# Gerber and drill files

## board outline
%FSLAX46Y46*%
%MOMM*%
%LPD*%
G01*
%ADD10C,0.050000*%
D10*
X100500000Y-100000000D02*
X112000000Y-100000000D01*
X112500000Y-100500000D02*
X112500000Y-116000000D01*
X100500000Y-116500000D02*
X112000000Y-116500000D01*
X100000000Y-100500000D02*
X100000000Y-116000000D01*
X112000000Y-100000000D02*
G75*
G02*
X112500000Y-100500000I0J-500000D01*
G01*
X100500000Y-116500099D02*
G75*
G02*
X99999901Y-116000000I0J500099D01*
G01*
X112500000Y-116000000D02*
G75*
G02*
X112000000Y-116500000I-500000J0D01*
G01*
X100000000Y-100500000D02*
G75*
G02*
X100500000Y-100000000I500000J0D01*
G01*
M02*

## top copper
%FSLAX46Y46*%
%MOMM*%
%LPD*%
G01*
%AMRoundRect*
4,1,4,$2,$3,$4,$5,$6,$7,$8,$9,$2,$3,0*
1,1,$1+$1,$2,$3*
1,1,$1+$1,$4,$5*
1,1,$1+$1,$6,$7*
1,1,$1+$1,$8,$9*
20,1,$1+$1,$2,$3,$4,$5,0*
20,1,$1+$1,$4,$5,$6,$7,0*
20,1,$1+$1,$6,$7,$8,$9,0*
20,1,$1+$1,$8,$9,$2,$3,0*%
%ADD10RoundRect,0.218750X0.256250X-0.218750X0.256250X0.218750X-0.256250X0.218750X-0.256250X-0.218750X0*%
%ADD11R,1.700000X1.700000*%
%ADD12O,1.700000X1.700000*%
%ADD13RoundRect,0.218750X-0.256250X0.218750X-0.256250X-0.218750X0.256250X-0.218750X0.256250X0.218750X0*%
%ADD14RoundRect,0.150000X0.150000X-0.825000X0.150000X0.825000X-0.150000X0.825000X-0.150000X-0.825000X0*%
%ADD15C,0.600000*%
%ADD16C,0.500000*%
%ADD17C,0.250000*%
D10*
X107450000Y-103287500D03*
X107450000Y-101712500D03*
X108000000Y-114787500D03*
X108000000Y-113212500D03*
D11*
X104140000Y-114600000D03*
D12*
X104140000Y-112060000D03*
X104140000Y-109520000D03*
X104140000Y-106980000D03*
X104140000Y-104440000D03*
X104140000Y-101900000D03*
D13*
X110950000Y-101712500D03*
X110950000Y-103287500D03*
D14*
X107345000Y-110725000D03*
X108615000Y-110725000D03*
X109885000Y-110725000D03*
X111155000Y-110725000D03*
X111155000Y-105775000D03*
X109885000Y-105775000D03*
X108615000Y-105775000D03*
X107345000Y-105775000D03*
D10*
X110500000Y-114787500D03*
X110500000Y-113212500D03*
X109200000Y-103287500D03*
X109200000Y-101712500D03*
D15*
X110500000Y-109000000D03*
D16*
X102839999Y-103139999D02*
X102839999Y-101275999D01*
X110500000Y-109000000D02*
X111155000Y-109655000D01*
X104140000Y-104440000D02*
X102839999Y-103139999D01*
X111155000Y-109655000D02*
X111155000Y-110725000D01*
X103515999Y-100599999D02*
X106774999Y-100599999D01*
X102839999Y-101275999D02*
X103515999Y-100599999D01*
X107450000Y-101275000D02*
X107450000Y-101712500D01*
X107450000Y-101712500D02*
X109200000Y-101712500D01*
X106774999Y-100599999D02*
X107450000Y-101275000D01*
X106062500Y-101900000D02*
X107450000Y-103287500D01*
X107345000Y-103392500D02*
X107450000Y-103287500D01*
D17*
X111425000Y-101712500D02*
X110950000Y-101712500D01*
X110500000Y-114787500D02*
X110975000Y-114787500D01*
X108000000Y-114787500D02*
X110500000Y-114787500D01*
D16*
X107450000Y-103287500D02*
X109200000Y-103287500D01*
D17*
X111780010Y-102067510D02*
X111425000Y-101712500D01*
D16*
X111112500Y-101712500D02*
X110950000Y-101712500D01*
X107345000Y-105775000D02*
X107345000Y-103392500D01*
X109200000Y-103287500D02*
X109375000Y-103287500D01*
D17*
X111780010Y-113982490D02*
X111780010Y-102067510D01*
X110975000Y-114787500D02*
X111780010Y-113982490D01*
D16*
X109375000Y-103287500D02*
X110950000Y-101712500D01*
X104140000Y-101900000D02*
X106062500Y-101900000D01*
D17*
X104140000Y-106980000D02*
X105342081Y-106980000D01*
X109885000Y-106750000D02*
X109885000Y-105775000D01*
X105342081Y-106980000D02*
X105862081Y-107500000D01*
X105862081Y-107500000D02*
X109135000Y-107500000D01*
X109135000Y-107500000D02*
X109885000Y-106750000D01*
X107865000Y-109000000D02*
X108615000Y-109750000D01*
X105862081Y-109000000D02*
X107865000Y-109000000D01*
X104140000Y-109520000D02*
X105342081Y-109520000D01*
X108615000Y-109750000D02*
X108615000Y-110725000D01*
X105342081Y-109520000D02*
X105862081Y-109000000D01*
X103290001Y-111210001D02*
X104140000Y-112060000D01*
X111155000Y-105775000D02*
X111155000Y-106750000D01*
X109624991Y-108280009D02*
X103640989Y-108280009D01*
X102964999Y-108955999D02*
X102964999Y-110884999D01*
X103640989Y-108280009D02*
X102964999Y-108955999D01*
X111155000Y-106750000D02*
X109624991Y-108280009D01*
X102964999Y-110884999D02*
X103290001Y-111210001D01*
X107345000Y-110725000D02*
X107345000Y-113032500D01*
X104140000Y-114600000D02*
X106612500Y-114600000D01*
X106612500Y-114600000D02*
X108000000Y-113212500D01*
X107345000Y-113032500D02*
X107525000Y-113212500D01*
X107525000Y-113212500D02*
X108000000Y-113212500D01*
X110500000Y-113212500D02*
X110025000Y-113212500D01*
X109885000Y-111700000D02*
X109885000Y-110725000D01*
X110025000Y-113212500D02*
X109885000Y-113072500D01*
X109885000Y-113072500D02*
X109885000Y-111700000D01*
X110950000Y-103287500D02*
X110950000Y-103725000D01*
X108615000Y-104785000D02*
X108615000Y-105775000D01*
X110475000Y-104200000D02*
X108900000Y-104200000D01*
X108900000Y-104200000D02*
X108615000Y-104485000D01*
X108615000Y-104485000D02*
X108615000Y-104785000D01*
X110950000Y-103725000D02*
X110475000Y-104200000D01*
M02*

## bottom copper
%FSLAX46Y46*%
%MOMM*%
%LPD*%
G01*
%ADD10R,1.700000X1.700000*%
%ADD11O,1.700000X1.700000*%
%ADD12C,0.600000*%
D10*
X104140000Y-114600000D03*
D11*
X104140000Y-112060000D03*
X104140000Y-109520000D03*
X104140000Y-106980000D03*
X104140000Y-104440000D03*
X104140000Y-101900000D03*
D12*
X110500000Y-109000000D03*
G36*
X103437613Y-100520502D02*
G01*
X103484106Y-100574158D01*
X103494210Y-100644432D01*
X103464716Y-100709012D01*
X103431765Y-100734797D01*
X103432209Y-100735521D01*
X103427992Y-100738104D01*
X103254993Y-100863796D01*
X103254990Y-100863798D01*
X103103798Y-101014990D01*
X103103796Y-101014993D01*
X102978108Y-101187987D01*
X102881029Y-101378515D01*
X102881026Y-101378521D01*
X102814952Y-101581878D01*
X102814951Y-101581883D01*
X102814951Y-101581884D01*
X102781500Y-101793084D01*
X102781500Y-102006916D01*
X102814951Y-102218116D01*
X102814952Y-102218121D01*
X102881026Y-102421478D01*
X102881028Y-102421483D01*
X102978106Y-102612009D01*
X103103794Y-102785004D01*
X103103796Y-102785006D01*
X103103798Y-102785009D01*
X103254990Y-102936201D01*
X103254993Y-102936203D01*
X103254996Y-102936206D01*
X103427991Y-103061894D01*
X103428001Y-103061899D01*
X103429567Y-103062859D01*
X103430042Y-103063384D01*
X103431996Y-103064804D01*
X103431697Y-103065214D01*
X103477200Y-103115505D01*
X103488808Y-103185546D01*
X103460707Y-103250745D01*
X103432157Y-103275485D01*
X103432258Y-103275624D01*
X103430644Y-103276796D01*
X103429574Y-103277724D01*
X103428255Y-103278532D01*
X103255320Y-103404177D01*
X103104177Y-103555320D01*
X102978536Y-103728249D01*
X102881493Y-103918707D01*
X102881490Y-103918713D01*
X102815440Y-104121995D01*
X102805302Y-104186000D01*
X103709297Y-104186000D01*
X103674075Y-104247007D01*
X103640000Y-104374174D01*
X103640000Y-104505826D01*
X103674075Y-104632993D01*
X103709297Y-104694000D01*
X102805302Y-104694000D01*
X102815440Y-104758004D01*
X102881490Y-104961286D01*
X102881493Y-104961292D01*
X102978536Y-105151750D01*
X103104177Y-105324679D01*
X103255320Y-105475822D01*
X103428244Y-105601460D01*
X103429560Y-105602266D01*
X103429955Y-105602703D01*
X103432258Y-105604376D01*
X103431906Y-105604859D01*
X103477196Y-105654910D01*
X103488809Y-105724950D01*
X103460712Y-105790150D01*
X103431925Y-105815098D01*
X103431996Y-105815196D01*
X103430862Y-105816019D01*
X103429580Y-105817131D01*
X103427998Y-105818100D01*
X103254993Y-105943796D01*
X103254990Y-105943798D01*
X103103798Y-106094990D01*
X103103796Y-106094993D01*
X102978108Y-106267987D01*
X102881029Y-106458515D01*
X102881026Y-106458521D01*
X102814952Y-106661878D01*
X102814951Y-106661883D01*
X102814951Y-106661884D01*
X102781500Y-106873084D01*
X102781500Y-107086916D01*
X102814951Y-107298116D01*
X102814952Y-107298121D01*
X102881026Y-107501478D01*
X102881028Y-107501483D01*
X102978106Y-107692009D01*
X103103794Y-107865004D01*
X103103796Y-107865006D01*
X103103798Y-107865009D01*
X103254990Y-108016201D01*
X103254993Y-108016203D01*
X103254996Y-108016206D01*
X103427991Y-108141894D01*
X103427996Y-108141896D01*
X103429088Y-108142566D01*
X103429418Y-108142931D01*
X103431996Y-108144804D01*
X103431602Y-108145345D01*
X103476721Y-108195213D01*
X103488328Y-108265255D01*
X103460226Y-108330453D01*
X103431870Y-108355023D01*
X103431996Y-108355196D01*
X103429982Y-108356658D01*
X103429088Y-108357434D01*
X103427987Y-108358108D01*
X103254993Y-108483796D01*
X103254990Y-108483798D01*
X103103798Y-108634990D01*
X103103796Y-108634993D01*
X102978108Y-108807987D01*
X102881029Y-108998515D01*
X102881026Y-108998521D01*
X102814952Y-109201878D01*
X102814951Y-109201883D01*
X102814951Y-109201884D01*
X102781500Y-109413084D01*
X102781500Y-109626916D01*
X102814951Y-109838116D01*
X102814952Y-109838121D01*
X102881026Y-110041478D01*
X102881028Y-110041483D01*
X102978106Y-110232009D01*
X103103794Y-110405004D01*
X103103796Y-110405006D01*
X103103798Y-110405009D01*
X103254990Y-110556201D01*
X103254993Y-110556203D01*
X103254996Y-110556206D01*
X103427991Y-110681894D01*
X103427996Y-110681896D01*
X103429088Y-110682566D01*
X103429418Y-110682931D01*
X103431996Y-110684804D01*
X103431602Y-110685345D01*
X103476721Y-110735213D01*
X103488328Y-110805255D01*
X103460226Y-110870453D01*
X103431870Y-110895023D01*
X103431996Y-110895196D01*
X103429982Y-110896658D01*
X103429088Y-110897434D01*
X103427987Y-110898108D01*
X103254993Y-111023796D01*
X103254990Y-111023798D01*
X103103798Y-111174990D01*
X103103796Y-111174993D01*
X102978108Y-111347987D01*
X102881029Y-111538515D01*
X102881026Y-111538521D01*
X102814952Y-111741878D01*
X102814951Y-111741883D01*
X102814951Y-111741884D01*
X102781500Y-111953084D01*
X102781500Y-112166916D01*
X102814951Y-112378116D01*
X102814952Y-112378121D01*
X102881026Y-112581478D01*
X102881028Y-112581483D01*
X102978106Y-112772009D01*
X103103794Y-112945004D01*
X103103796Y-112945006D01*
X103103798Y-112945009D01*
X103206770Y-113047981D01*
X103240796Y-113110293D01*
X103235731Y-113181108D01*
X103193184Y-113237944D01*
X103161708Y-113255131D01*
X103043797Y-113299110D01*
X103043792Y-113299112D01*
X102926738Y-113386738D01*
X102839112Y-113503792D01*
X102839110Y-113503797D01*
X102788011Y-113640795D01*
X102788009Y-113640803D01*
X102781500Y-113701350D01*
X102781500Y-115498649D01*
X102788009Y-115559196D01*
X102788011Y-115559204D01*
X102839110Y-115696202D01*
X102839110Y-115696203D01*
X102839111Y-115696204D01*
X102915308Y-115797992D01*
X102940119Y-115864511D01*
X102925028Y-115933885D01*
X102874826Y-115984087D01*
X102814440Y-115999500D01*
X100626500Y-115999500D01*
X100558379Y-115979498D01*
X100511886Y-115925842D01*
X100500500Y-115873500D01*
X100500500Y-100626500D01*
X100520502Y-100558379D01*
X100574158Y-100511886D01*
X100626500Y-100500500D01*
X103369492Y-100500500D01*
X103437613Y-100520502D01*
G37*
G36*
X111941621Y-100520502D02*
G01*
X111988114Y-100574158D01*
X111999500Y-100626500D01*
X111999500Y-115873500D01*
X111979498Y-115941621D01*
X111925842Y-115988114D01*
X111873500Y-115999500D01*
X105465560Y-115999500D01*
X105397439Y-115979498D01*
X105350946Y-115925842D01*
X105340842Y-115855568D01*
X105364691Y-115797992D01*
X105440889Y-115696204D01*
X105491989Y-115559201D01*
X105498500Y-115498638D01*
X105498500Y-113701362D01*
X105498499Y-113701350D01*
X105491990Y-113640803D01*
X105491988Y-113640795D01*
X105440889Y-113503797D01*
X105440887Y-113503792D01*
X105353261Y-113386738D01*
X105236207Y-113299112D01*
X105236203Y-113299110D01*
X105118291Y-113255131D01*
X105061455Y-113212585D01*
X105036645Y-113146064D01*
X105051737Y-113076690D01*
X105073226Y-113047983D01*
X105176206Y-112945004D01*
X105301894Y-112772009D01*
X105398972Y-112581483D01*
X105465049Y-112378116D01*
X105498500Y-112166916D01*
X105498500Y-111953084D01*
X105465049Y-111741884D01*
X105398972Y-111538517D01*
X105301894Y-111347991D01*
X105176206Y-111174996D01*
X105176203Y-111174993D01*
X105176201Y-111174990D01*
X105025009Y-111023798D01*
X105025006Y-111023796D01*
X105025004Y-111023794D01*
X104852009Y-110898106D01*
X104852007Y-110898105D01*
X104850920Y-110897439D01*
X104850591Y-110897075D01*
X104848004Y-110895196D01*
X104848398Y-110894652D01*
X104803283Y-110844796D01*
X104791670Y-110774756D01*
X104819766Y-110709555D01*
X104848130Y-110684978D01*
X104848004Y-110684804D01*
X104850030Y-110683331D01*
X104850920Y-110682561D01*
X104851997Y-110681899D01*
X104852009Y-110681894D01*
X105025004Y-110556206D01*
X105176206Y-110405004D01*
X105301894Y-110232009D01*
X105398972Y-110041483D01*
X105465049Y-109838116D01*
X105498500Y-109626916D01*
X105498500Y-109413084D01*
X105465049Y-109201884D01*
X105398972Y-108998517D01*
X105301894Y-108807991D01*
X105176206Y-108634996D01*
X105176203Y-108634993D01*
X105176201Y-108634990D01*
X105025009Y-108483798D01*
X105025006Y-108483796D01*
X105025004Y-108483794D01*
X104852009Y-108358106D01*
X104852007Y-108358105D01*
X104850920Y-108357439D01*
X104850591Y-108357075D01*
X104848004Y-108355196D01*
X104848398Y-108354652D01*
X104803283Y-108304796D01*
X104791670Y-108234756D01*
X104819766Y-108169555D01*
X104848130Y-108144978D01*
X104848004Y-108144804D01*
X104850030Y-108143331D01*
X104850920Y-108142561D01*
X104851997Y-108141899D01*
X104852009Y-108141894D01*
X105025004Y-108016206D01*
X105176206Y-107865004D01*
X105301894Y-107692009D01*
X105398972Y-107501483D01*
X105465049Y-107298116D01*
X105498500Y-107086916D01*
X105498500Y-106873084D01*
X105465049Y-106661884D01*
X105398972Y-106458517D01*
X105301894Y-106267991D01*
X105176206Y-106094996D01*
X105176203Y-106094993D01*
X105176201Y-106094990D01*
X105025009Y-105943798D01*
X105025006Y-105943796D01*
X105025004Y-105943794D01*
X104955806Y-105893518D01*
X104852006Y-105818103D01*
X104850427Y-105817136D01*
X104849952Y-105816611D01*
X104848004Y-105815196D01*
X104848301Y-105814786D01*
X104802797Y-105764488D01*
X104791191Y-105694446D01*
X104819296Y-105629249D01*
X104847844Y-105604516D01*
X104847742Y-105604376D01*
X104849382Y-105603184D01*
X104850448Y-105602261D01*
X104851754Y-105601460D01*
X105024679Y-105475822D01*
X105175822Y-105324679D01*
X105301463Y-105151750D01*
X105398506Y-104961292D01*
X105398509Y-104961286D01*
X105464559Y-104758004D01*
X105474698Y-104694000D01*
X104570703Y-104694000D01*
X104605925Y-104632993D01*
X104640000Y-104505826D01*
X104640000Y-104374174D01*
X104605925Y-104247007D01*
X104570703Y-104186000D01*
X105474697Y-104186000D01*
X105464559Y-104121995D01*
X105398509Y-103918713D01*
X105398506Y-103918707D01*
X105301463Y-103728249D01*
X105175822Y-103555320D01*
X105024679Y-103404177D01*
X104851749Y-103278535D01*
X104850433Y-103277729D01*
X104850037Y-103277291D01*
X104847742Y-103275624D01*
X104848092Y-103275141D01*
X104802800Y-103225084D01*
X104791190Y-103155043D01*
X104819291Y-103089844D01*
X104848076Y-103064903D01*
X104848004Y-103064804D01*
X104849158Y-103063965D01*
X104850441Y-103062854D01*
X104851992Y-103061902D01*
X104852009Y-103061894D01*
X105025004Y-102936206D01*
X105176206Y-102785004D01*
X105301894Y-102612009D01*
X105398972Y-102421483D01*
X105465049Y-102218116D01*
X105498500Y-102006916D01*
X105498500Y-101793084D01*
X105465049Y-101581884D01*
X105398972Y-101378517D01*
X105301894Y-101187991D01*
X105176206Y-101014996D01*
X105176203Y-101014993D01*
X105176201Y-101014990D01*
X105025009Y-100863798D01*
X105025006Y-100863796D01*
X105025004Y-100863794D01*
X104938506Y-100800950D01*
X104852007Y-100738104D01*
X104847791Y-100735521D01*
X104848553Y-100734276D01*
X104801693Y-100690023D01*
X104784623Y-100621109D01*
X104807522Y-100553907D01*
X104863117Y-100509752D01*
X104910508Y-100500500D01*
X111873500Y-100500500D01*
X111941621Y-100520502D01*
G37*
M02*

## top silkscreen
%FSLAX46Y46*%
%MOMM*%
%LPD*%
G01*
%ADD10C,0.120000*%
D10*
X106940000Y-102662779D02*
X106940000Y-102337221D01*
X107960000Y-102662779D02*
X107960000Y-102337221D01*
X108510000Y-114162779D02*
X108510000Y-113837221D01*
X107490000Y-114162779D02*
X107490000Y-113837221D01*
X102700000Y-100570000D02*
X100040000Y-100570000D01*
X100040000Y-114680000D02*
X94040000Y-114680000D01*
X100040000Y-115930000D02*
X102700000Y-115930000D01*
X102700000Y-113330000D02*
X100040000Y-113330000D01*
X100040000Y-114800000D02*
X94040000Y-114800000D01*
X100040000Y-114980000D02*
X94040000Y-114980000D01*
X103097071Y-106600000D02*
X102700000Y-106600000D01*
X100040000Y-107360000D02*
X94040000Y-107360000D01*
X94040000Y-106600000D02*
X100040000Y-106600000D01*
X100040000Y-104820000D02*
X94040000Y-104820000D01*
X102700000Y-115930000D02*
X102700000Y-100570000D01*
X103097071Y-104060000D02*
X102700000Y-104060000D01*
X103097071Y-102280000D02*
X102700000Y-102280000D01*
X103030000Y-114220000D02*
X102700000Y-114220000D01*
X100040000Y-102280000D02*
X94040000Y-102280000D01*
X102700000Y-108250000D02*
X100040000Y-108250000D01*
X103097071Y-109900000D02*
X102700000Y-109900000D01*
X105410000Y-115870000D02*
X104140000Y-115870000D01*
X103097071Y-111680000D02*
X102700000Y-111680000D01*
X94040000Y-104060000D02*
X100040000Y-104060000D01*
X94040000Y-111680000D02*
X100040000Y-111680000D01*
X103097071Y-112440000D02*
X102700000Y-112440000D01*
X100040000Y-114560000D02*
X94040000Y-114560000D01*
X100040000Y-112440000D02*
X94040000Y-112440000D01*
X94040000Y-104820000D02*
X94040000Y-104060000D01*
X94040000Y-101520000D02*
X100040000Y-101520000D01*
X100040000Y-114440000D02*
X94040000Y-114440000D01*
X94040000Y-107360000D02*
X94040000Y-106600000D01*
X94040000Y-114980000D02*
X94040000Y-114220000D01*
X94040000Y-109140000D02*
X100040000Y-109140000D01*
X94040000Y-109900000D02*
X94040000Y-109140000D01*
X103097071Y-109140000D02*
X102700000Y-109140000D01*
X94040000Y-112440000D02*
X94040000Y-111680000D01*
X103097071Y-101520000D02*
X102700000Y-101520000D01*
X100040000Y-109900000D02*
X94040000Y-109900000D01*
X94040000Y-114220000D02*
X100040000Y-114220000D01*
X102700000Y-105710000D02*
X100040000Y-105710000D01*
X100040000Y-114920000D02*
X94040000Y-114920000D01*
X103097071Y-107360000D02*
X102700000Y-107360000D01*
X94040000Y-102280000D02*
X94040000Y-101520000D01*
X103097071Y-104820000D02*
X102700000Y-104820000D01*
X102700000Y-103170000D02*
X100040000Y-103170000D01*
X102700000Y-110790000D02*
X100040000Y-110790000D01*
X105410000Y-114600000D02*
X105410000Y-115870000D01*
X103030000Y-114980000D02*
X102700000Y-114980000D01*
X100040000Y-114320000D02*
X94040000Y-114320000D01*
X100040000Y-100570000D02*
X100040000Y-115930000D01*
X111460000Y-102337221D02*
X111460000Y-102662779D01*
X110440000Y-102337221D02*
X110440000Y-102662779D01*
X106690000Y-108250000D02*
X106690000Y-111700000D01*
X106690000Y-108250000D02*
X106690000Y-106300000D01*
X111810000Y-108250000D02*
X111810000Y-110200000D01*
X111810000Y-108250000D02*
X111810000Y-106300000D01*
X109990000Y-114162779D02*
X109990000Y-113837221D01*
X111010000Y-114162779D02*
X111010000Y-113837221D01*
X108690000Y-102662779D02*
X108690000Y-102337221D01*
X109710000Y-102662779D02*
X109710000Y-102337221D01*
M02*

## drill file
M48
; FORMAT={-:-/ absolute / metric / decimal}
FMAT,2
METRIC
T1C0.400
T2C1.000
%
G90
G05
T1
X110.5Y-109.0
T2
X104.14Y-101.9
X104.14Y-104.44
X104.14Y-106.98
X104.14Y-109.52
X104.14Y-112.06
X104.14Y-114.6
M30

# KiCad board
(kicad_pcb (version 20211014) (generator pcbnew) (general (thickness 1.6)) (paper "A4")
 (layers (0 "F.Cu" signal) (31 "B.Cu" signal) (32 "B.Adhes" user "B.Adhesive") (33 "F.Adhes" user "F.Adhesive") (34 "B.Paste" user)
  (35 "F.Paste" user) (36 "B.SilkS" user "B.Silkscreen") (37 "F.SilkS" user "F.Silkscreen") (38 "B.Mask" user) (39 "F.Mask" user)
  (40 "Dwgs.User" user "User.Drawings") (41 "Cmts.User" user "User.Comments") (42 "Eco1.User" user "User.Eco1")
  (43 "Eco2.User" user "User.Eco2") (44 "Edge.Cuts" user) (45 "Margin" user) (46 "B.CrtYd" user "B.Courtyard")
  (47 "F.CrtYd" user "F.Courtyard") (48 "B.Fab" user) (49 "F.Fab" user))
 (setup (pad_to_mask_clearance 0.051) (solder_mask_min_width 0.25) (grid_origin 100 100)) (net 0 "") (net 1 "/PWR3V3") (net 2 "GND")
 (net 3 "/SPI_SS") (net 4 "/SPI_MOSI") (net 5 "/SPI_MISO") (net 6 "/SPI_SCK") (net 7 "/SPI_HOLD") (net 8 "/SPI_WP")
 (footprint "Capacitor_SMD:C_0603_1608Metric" (layer "F.Cu") (at 107.45 102.5 90)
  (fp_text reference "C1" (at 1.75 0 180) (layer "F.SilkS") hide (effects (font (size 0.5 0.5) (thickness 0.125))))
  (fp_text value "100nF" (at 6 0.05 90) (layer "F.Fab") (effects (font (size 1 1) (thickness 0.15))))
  (fp_line (start -0.162779 -0.51) (end 0.162779 -0.51) (layer "F.SilkS") (width 0.12))
  (fp_line (start -0.162779 0.51) (end 0.162779 0.51) (layer "F.SilkS") (width 0.12))
  (pad "1" smd roundrect locked (at -0.7875 0 90) (size 0.875 0.95) (layers "F.Cu" "F.Paste" "F.Mask") (roundrect_rratio 0.25)
   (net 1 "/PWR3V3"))
  (pad "2" smd roundrect locked (at 0.7875 0 90) (size 0.875 0.95) (layers "F.Cu" "F.Paste" "F.Mask") (roundrect_rratio 0.25) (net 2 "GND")))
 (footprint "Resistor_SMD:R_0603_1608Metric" (layer "F.Cu") (at 108 114 90)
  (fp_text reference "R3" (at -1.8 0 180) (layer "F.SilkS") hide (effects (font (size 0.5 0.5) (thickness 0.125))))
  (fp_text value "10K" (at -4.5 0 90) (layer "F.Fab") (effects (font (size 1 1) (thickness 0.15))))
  (fp_line (start -0.162779 0.51) (end 0.162779 0.51) (layer "F.SilkS") (width 0.12))
  (fp_line (start -0.162779 -0.51) (end 0.162779 -0.51) (layer "F.SilkS") (width 0.12))
  (pad "1" smd roundrect locked (at -0.7875 0 90) (size 0.875 0.95) (layers "F.Cu" "F.Paste" "F.Mask") (roundrect_rratio 0.25)
   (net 1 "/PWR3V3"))
  (pad "2" smd roundrect locked (at 0.7875 0 90) (size 0.875 0.95) (layers "F.Cu" "F.Paste" "F.Mask") (roundrect_rratio 0.25)
   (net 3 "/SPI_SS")))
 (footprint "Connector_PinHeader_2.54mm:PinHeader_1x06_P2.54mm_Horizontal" (layer "F.Cu") (at 104.14 114.6 180)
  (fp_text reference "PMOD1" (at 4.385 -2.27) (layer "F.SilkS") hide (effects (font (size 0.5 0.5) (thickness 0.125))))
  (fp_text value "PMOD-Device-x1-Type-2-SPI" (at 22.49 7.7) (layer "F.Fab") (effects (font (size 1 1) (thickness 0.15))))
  (fp_line (start 1.44 14.03) (end 4.1 14.03) (layer "F.SilkS") (width 0.12))
  (fp_line (start 4.1 -0.08) (end 10.1 -0.08) (layer "F.SilkS") (width 0.12))
  (fp_line (start 4.1 -1.33) (end 1.44 -1.33) (layer "F.SilkS") (width 0.12))
  (fp_line (start 1.44 1.27) (end 4.1 1.27) (layer "F.SilkS") (width 0.12))
  (fp_line (start 4.1 -0.2) (end 10.1 -0.2) (layer "F.SilkS") (width 0.12))
  (fp_line (start 4.1 -0.38) (end 10.1 -0.38) (layer "F.SilkS") (width 0.12))
  (fp_line (start 1.042929 8) (end 1.44 8) (layer "F.SilkS") (width 0.12))
  (fp_line (start 4.1 7.24) (end 10.1 7.24) (layer "F.SilkS") (width 0.12))
  (fp_line (start 10.1 8) (end 4.1 8) (layer "F.SilkS") (width 0.12))
  (fp_line (start 4.1 9.78) (end 10.1 9.78) (layer "F.SilkS") (width 0.12))
  (fp_line (start 1.44 -1.33) (end 1.44 14.03) (layer "F.SilkS") (width 0.12))
  (fp_line (start 1.042929 10.54) (end 1.44 10.54) (layer "F.SilkS") (width 0.12))
  (fp_line (start 1.042929 12.32) (end 1.44 12.32) (layer "F.SilkS") (width 0.12))
  (fp_line (start 1.11 0.38) (end 1.44 0.38) (layer "F.SilkS") (width 0.12))
  (fp_line (start 4.1 12.32) (end 10.1 12.32) (layer "F.SilkS") (width 0.12))
  (fp_line (start 1.44 6.35) (end 4.1 6.35) (layer "F.SilkS") (width 0.12))
  (fp_line (start 1.042929 4.7) (end 1.44 4.7) (layer "F.SilkS") (width 0.12))
  (fp_line (start -1.27 -1.27) (end 0 -1.27) (layer "F.SilkS") (width 0.12))
  (fp_line (start 1.042929 2.92) (end 1.44 2.92) (layer "F.SilkS") (width 0.12))
  (fp_line (start 10.1 10.54) (end 4.1 10.54) (layer "F.SilkS") (width 0.12))
  (fp_line (start 10.1 2.92) (end 4.1 2.92) (layer "F.SilkS") (width 0.12))
  (fp_line (start 1.042929 2.16) (end 1.44 2.16) (layer "F.SilkS") (width 0.12))
  (fp_line (start 4.1 0.04) (end 10.1 0.04) (layer "F.SilkS") (width 0.12))
  (fp_line (start 4.1 2.16) (end 10.1 2.16) (layer "F.SilkS") (width 0.12))
  (fp_line (start 10.1 9.78) (end 10.1 10.54) (layer "F.SilkS") (width 0.12))
  (fp_line (start 10.1 13.08) (end 4.1 13.08) (layer "F.SilkS") (width 0.12))
  (fp_line (start 4.1 0.16) (end 10.1 0.16) (layer "F.SilkS") (width 0.12))
  (fp_line (start 10.1 7.24) (end 10.1 8) (layer "F.SilkS") (width 0.12))
  (fp_line (start 10.1 -0.38) (end 10.1 0.38) (layer "F.SilkS") (width 0.12))
  (fp_line (start 10.1 5.46) (end 4.1 5.46) (layer "F.SilkS") (width 0.12))
  (fp_line (start 10.1 4.7) (end 10.1 5.46) (layer "F.SilkS") (width 0.12))
  (fp_line (start 1.042929 5.46) (end 1.44 5.46) (layer "F.SilkS") (width 0.12))
  (fp_line (start 10.1 2.16) (end 10.1 2.92) (layer "F.SilkS") (width 0.12))
  (fp_line (start 1.042929 13.08) (end 1.44 13.08) (layer "F.SilkS") (width 0.12))
  (fp_line (start 4.1 4.7) (end 10.1 4.7) (layer "F.SilkS") (width 0.12))
  (fp_line (start 10.1 0.38) (end 4.1 0.38) (layer "F.SilkS") (width 0.12))
  (fp_line (start 1.44 8.89) (end 4.1 8.89) (layer "F.SilkS") (width 0.12))
  (fp_line (start 4.1 -0.32) (end 10.1 -0.32) (layer "F.SilkS") (width 0.12))
  (fp_line (start 1.042929 7.24) (end 1.44 7.24) (layer "F.SilkS") (width 0.12))
  (fp_line (start 10.1 12.32) (end 10.1 13.08) (layer "F.SilkS") (width 0.12))
  (fp_line (start 1.042929 9.78) (end 1.44 9.78) (layer "F.SilkS") (width 0.12))
  (fp_line (start 1.44 11.43) (end 4.1 11.43) (layer "F.SilkS") (width 0.12))
  (fp_line (start 1.44 3.81) (end 4.1 3.81) (layer "F.SilkS") (width 0.12))
  (fp_line (start -1.27 0) (end -1.27 -1.27) (layer "F.SilkS") (width 0.12))
  (fp_line (start 1.11 -0.38) (end 1.44 -0.38) (layer "F.SilkS") (width 0.12))
  (fp_line (start 4.1 0.28) (end 10.1 0.28) (layer "F.SilkS") (width 0.12))
  (fp_line (start 4.1 14.03) (end 4.1 -1.33) (layer "F.SilkS") (width 0.12))
  (pad "1" thru_hole rect locked (at 0 0 180) (size 1.7 1.7) (drill 1) (layers *.Cu *.Mask) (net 3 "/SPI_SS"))
  (pad "2" thru_hole oval locked (at 0 2.54 180) (size 1.7 1.7) (drill 1) (layers *.Cu *.Mask) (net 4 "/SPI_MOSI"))
  (pad "3" thru_hole oval locked (at 0 5.08 180) (size 1.7 1.7) (drill 1) (layers *.Cu *.Mask) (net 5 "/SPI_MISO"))
  (pad "4" thru_hole oval locked (at 0 7.62 180) (size 1.7 1.7) (drill 1) (layers *.Cu *.Mask) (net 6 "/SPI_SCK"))
  (pad "5" thru_hole oval locked (at 0 10.16 180) (size 1.7 1.7) (drill 1) (layers *.Cu *.Mask) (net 2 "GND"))
  (pad "6" thru_hole oval locked (at 0 12.7 180) (size 1.7 1.7) (drill 1) (layers *.Cu *.Mask) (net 1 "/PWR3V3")))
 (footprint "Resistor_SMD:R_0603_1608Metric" (layer "F.Cu") (at 110.95 102.5 -90)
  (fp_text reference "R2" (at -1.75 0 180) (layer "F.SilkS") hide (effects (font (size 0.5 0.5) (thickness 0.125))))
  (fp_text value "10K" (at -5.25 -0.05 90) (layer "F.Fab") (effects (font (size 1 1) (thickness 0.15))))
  (fp_line (start -0.162779 -0.51) (end 0.162779 -0.51) (layer "F.SilkS") (width 0.12))
  (fp_line (start -0.162779 0.51) (end 0.162779 0.51) (layer "F.SilkS") (width 0.12))
  (pad "1" smd roundrect locked (at -0.7875 0 270) (size 0.875 0.95) (layers "F.Cu" "F.Paste" "F.Mask") (roundrect_rratio 0.25)
   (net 1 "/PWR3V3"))
  (pad "2" smd roundrect locked (at 0.7875 0 270) (size 0.875 0.95) (layers "F.Cu" "F.Paste" "F.Mask") (roundrect_rratio 0.25)
   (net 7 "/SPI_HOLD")))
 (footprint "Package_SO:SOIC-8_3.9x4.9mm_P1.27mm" (layer "F.Cu") (at 109.25 108.25 90)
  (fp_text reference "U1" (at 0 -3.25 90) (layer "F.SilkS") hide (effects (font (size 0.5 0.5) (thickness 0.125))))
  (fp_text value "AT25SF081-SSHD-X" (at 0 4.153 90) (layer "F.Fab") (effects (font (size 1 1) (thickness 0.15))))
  (fp_line (start 0 -2.56) (end -3.45 -2.56) (layer "F.SilkS") (width 0.12))
  (fp_line (start 0 -2.56) (end 1.95 -2.56) (layer "F.SilkS") (width 0.12))
  (fp_line (start 0 2.56) (end -1.95 2.56) (layer "F.SilkS") (width 0.12))
  (fp_line (start 0 2.56) (end 1.95 2.56) (layer "F.SilkS") (width 0.12))
  (pad "1" smd roundrect locked (at -2.475 -1.905 90) (size 1.95 0.6) (layers "F.Cu" "F.Paste" "F.Mask") (roundrect_rratio 0.25)
   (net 3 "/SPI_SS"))
  (pad "2" smd roundrect locked (at -2.475 -0.635 90) (size 1.95 0.6) (layers "F.Cu" "F.Paste" "F.Mask") (roundrect_rratio 0.25)
   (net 5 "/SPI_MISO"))
  (pad "3" smd roundrect locked (at -2.475 0.635 90) (size 1.95 0.6) (layers "F.Cu" "F.Paste" "F.Mask") (roundrect_rratio 0.25)
   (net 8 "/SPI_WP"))
  (pad "4" smd roundrect locked (at -2.475 1.905 90) (size 1.95 0.6) (layers "F.Cu" "F.Paste" "F.Mask") (roundrect_rratio 0.25)
   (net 2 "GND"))
  (pad "5" smd roundrect locked (at 2.475 1.905 90) (size 1.95 0.6) (layers "F.Cu" "F.Paste" "F.Mask") (roundrect_rratio 0.25)
   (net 4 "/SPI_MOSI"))
  (pad "6" smd roundrect locked (at 2.475 0.635 90) (size 1.95 0.6) (layers "F.Cu" "F.Paste" "F.Mask") (roundrect_rratio 0.25)
   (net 6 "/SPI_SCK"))
  (pad "7" smd roundrect locked (at 2.475 -0.635 90) (size 1.95 0.6) (layers "F.Cu" "F.Paste" "F.Mask") (roundrect_rratio 0.25)
   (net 7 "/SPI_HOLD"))
  (pad "8" smd roundrect locked (at 2.475 -1.905 90) (size 1.95 0.6) (layers "F.Cu" "F.Paste" "F.Mask") (roundrect_rratio 0.25)
   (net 1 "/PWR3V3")))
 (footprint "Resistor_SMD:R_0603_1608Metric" (layer "F.Cu") (at 110.5 114 90)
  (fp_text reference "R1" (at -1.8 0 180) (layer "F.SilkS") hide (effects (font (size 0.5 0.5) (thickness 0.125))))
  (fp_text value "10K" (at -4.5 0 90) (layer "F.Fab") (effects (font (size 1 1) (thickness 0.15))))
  (fp_line (start -0.162779 -0.51) (end 0.162779 -0.51) (layer "F.SilkS") (width 0.12))
  (fp_line (start -0.162779 0.51) (end 0.162779 0.51) (layer "F.SilkS") (width 0.12))
  (pad "1" smd roundrect locked (at -0.7875 0 90) (size 0.875 0.95) (layers "F.Cu" "F.Paste" "F.Mask") (roundrect_rratio 0.25)
   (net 1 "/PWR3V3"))
  (pad "2" smd roundrect locked (at 0.7875 0 90) (size 0.875 0.95) (layers "F.Cu" "F.Paste" "F.Mask") (roundrect_rratio 0.25)
   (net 8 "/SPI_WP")))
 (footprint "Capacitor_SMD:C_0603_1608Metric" (layer "F.Cu") (at 109.2 102.5 90)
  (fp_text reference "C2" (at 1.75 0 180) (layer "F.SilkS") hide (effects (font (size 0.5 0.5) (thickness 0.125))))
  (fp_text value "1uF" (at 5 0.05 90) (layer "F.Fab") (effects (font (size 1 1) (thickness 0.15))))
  (fp_line (start -0.162779 -0.51) (end 0.162779 -0.51) (layer "F.SilkS") (width 0.12))
  (fp_line (start -0.162779 0.51) (end 0.162779 0.51) (layer "F.SilkS") (width 0.12))
  (pad "1" smd roundrect locked (at -0.7875 0 90) (size 0.875 0.95) (layers "F.Cu" "F.Paste" "F.Mask") (roundrect_rratio 0.25)
   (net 1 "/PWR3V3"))
  (pad "2" smd roundrect locked (at 0.7875 0 90) (size 0.875 0.95) (layers "F.Cu" "F.Paste" "F.Mask") (roundrect_rratio 0.25) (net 2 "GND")))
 (gr_line (start 100.5 100) (end 112 100) (layer "Edge.Cuts") (width 0.05))
 (gr_line (start 112.5 100.5) (end 112.5 116) (layer "Edge.Cuts") (width 0.05))
 (gr_line (start 100.5 116.5) (end 112 116.5) (layer "Edge.Cuts") (width 0.05))
 (gr_line (start 100 100.5) (end 100 116) (layer "Edge.Cuts") (width 0.05))
 (gr_arc (start 112 100) (mid 112.353553 100.146447) (end 112.5 100.5) (layer "Edge.Cuts") (width 0.05))
 (gr_arc (start 100.5 116.500099) (mid 100.146377 116.353623) (end 99.999901 116) (layer "Edge.Cuts") (width 0.05))
 (gr_arc (start 112.5 116) (mid 112.353553 116.353553) (end 112 116.5) (layer "Edge.Cuts") (width 0.05))
 (gr_arc (start 100 100.5) (mid 100.146447 100.146447) (end 100.5 100) (layer "Edge.Cuts") (width 0.05))
 (segment (start 102.839999 103.139999) (end 102.839999 101.275999) (width 0.5) (layer "F.Cu") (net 2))
 (segment (start 110.5 109) (end 111.155 109.655) (width 0.5) (layer "F.Cu") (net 2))
 (segment (start 104.14 104.44) (end 102.839999 103.139999) (width 0.5) (layer "F.Cu") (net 2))
 (segment (start 111.155 109.655) (end 111.155 110.725) (width 0.5) (layer "F.Cu") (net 2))
 (segment (start 103.515999 100.599999) (end 106.774999 100.599999) (width 0.5) (layer "F.Cu") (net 2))
 (segment (start 102.839999 101.275999) (end 103.515999 100.599999) (width 0.5) (layer "F.Cu") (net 2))
 (segment (start 107.45 101.275) (end 107.45 101.7125) (width 0.5) (layer "F.Cu") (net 2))
 (segment (start 107.45 101.7125) (end 109.2 101.7125) (width 0.5) (layer "F.Cu") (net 2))
 (segment (start 106.774999 100.599999) (end 107.45 101.275) (width 0.5) (layer "F.Cu") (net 2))
 (via (at 110.5 109) (size 0.6) (drill 0.4) (layers "F.Cu" "B.Cu") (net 2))
 (segment (start 106.0625 101.9) (end 107.45 103.2875) (width 0.5) (layer "F.Cu") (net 1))
 (segment (start 107.345 103.3925) (end 107.45 103.2875) (width 0.5) (layer "F.Cu") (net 1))
 (segment (start 111.425 101.7125) (end 110.95 101.7125) (width 0.25) (layer "F.Cu") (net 1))
 (segment (start 110.5 114.7875) (end 110.975 114.7875) (width 0.25) (layer "F.Cu") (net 1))
 (segment (start 108 114.7875) (end 110.5 114.7875) (width 0.25) (layer "F.Cu") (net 1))
 (segment (start 107.45 103.2875) (end 109.2 103.2875) (width 0.5) (layer "F.Cu") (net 1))
 (segment (start 111.78001 102.06751) (end 111.425 101.7125) (width 0.25) (layer "F.Cu") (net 1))
 (segment (start 111.1125 101.7125) (end 110.95 101.7125) (width 0.5) (layer "F.Cu") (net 1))
 (segment (start 107.345 105.775) (end 107.345 103.3925) (width 0.5) (layer "F.Cu") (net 1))
 (segment (start 109.2 103.2875) (end 109.375 103.2875) (width 0.5) (layer "F.Cu") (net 1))
 (segment (start 111.78001 113.98249) (end 111.78001 102.06751) (width 0.25) (layer "F.Cu") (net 1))
 (segment (start 110.975 114.7875) (end 111.78001 113.98249) (width 0.25) (layer "F.Cu") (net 1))
 (segment (start 109.375 103.2875) (end 110.95 101.7125) (width 0.5) (layer "F.Cu") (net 1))
 (segment (start 104.14 101.9) (end 106.0625 101.9) (width 0.5) (layer "F.Cu") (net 1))
 (segment (start 104.14 106.98) (end 105.342081 106.98) (width 0.25) (layer "F.Cu") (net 6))
 (segment (start 109.885 106.75) (end 109.885 105.775) (width 0.25) (layer "F.Cu") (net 6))
 (segment (start 105.342081 106.98) (end 105.862081 107.5) (width 0.25) (layer "F.Cu") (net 6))
 (segment (start 105.862081 107.5) (end 109.135 107.5) (width 0.25) (layer "F.Cu") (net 6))
 (segment (start 109.135 107.5) (end 109.885 106.75) (width 0.25) (layer "F.Cu") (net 6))
 (segment (start 107.865 109) (end 108.615 109.75) (width 0.25) (layer "F.Cu") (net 5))
 (segment (start 105.862081 109) (end 107.865 109) (width 0.25) (layer "F.Cu") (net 5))
 (segment (start 104.14 109.52) (end 105.342081 109.52) (width 0.25) (layer "F.Cu") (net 5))
 (segment (start 108.615 109.75) (end 108.615 110.725) (width 0.25) (layer "F.Cu") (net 5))
 (segment (start 105.342081 109.52) (end 105.862081 109) (width 0.25) (layer "F.Cu") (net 5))
 (segment (start 103.290001 111.210001) (end 104.14 112.06) (width 0.25) (layer "F.Cu") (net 4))
 (segment (start 111.155 105.775) (end 111.155 106.75) (width 0.25) (layer "F.Cu") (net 4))
 (segment (start 109.624991 108.280009) (end 103.640989 108.280009) (width 0.25) (layer "F.Cu") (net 4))
 (segment (start 102.964999 108.955999) (end 102.964999 110.884999) (width 0.25) (layer "F.Cu") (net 4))
 (segment (start 103.640989 108.280009) (end 102.964999 108.955999) (width 0.25) (layer "F.Cu") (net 4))
 (segment (start 111.155 106.75) (end 109.624991 108.280009) (width 0.25) (layer "F.Cu") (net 4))
 (segment (start 102.964999 110.884999) (end 103.290001 111.210001) (width 0.25) (layer "F.Cu") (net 4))
 (segment (start 107.345 110.725) (end 107.345 113.0325) (width 0.25) (layer "F.Cu") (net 3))
 (segment (start 104.14 114.6) (end 106.6125 114.6) (width 0.25) (layer "F.Cu") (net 3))
 (segment (start 106.6125 114.6) (end 108 113.2125) (width 0.25) (layer "F.Cu") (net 3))
 (segment (start 107.345 113.0325) (end 107.525 113.2125) (width 0.25) (layer "F.Cu") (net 3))
 (segment (start 107.525 113.2125) (end 108 113.2125) (width 0.25) (layer "F.Cu") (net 3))
 (segment (start 110.5 113.2125) (end 110.025 113.2125) (width 0.25) (layer "F.Cu") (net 8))
 (segment (start 109.885 111.7) (end 109.885 110.725) (width 0.25) (layer "F.Cu") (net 8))
 (segment (start 110.025 113.2125) (end 109.885 113.0725) (width 0.25) (layer "F.Cu") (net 8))
 (segment (start 109.885 113.0725) (end 109.885 111.7) (width 0.25) (layer "F.Cu") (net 8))
 (segment (start 110.95 103.2875) (end 110.95 103.725) (width 0.25) (layer "F.Cu") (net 7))
 (segment (start 108.615 104.785) (end 108.615 105.775) (width 0.25) (layer "F.Cu") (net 7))
 (segment (start 110.475 104.2) (end 108.9 104.2) (width 0.25) (layer "F.Cu") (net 7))
 (segment (start 108.9 104.2) (end 108.615 104.485) (width 0.25) (layer "F.Cu") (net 7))
 (segment (start 108.615 104.485) (end 108.615 104.785) (width 0.25) (layer "F.Cu") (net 7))
 (segment (start 110.95 103.725) (end 110.475 104.2) (width 0.25) (layer "F.Cu") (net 7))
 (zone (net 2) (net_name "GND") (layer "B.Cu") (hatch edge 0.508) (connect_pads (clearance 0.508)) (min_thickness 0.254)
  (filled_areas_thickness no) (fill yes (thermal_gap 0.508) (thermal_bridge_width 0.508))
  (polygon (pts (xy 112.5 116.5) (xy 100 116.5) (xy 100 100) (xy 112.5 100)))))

